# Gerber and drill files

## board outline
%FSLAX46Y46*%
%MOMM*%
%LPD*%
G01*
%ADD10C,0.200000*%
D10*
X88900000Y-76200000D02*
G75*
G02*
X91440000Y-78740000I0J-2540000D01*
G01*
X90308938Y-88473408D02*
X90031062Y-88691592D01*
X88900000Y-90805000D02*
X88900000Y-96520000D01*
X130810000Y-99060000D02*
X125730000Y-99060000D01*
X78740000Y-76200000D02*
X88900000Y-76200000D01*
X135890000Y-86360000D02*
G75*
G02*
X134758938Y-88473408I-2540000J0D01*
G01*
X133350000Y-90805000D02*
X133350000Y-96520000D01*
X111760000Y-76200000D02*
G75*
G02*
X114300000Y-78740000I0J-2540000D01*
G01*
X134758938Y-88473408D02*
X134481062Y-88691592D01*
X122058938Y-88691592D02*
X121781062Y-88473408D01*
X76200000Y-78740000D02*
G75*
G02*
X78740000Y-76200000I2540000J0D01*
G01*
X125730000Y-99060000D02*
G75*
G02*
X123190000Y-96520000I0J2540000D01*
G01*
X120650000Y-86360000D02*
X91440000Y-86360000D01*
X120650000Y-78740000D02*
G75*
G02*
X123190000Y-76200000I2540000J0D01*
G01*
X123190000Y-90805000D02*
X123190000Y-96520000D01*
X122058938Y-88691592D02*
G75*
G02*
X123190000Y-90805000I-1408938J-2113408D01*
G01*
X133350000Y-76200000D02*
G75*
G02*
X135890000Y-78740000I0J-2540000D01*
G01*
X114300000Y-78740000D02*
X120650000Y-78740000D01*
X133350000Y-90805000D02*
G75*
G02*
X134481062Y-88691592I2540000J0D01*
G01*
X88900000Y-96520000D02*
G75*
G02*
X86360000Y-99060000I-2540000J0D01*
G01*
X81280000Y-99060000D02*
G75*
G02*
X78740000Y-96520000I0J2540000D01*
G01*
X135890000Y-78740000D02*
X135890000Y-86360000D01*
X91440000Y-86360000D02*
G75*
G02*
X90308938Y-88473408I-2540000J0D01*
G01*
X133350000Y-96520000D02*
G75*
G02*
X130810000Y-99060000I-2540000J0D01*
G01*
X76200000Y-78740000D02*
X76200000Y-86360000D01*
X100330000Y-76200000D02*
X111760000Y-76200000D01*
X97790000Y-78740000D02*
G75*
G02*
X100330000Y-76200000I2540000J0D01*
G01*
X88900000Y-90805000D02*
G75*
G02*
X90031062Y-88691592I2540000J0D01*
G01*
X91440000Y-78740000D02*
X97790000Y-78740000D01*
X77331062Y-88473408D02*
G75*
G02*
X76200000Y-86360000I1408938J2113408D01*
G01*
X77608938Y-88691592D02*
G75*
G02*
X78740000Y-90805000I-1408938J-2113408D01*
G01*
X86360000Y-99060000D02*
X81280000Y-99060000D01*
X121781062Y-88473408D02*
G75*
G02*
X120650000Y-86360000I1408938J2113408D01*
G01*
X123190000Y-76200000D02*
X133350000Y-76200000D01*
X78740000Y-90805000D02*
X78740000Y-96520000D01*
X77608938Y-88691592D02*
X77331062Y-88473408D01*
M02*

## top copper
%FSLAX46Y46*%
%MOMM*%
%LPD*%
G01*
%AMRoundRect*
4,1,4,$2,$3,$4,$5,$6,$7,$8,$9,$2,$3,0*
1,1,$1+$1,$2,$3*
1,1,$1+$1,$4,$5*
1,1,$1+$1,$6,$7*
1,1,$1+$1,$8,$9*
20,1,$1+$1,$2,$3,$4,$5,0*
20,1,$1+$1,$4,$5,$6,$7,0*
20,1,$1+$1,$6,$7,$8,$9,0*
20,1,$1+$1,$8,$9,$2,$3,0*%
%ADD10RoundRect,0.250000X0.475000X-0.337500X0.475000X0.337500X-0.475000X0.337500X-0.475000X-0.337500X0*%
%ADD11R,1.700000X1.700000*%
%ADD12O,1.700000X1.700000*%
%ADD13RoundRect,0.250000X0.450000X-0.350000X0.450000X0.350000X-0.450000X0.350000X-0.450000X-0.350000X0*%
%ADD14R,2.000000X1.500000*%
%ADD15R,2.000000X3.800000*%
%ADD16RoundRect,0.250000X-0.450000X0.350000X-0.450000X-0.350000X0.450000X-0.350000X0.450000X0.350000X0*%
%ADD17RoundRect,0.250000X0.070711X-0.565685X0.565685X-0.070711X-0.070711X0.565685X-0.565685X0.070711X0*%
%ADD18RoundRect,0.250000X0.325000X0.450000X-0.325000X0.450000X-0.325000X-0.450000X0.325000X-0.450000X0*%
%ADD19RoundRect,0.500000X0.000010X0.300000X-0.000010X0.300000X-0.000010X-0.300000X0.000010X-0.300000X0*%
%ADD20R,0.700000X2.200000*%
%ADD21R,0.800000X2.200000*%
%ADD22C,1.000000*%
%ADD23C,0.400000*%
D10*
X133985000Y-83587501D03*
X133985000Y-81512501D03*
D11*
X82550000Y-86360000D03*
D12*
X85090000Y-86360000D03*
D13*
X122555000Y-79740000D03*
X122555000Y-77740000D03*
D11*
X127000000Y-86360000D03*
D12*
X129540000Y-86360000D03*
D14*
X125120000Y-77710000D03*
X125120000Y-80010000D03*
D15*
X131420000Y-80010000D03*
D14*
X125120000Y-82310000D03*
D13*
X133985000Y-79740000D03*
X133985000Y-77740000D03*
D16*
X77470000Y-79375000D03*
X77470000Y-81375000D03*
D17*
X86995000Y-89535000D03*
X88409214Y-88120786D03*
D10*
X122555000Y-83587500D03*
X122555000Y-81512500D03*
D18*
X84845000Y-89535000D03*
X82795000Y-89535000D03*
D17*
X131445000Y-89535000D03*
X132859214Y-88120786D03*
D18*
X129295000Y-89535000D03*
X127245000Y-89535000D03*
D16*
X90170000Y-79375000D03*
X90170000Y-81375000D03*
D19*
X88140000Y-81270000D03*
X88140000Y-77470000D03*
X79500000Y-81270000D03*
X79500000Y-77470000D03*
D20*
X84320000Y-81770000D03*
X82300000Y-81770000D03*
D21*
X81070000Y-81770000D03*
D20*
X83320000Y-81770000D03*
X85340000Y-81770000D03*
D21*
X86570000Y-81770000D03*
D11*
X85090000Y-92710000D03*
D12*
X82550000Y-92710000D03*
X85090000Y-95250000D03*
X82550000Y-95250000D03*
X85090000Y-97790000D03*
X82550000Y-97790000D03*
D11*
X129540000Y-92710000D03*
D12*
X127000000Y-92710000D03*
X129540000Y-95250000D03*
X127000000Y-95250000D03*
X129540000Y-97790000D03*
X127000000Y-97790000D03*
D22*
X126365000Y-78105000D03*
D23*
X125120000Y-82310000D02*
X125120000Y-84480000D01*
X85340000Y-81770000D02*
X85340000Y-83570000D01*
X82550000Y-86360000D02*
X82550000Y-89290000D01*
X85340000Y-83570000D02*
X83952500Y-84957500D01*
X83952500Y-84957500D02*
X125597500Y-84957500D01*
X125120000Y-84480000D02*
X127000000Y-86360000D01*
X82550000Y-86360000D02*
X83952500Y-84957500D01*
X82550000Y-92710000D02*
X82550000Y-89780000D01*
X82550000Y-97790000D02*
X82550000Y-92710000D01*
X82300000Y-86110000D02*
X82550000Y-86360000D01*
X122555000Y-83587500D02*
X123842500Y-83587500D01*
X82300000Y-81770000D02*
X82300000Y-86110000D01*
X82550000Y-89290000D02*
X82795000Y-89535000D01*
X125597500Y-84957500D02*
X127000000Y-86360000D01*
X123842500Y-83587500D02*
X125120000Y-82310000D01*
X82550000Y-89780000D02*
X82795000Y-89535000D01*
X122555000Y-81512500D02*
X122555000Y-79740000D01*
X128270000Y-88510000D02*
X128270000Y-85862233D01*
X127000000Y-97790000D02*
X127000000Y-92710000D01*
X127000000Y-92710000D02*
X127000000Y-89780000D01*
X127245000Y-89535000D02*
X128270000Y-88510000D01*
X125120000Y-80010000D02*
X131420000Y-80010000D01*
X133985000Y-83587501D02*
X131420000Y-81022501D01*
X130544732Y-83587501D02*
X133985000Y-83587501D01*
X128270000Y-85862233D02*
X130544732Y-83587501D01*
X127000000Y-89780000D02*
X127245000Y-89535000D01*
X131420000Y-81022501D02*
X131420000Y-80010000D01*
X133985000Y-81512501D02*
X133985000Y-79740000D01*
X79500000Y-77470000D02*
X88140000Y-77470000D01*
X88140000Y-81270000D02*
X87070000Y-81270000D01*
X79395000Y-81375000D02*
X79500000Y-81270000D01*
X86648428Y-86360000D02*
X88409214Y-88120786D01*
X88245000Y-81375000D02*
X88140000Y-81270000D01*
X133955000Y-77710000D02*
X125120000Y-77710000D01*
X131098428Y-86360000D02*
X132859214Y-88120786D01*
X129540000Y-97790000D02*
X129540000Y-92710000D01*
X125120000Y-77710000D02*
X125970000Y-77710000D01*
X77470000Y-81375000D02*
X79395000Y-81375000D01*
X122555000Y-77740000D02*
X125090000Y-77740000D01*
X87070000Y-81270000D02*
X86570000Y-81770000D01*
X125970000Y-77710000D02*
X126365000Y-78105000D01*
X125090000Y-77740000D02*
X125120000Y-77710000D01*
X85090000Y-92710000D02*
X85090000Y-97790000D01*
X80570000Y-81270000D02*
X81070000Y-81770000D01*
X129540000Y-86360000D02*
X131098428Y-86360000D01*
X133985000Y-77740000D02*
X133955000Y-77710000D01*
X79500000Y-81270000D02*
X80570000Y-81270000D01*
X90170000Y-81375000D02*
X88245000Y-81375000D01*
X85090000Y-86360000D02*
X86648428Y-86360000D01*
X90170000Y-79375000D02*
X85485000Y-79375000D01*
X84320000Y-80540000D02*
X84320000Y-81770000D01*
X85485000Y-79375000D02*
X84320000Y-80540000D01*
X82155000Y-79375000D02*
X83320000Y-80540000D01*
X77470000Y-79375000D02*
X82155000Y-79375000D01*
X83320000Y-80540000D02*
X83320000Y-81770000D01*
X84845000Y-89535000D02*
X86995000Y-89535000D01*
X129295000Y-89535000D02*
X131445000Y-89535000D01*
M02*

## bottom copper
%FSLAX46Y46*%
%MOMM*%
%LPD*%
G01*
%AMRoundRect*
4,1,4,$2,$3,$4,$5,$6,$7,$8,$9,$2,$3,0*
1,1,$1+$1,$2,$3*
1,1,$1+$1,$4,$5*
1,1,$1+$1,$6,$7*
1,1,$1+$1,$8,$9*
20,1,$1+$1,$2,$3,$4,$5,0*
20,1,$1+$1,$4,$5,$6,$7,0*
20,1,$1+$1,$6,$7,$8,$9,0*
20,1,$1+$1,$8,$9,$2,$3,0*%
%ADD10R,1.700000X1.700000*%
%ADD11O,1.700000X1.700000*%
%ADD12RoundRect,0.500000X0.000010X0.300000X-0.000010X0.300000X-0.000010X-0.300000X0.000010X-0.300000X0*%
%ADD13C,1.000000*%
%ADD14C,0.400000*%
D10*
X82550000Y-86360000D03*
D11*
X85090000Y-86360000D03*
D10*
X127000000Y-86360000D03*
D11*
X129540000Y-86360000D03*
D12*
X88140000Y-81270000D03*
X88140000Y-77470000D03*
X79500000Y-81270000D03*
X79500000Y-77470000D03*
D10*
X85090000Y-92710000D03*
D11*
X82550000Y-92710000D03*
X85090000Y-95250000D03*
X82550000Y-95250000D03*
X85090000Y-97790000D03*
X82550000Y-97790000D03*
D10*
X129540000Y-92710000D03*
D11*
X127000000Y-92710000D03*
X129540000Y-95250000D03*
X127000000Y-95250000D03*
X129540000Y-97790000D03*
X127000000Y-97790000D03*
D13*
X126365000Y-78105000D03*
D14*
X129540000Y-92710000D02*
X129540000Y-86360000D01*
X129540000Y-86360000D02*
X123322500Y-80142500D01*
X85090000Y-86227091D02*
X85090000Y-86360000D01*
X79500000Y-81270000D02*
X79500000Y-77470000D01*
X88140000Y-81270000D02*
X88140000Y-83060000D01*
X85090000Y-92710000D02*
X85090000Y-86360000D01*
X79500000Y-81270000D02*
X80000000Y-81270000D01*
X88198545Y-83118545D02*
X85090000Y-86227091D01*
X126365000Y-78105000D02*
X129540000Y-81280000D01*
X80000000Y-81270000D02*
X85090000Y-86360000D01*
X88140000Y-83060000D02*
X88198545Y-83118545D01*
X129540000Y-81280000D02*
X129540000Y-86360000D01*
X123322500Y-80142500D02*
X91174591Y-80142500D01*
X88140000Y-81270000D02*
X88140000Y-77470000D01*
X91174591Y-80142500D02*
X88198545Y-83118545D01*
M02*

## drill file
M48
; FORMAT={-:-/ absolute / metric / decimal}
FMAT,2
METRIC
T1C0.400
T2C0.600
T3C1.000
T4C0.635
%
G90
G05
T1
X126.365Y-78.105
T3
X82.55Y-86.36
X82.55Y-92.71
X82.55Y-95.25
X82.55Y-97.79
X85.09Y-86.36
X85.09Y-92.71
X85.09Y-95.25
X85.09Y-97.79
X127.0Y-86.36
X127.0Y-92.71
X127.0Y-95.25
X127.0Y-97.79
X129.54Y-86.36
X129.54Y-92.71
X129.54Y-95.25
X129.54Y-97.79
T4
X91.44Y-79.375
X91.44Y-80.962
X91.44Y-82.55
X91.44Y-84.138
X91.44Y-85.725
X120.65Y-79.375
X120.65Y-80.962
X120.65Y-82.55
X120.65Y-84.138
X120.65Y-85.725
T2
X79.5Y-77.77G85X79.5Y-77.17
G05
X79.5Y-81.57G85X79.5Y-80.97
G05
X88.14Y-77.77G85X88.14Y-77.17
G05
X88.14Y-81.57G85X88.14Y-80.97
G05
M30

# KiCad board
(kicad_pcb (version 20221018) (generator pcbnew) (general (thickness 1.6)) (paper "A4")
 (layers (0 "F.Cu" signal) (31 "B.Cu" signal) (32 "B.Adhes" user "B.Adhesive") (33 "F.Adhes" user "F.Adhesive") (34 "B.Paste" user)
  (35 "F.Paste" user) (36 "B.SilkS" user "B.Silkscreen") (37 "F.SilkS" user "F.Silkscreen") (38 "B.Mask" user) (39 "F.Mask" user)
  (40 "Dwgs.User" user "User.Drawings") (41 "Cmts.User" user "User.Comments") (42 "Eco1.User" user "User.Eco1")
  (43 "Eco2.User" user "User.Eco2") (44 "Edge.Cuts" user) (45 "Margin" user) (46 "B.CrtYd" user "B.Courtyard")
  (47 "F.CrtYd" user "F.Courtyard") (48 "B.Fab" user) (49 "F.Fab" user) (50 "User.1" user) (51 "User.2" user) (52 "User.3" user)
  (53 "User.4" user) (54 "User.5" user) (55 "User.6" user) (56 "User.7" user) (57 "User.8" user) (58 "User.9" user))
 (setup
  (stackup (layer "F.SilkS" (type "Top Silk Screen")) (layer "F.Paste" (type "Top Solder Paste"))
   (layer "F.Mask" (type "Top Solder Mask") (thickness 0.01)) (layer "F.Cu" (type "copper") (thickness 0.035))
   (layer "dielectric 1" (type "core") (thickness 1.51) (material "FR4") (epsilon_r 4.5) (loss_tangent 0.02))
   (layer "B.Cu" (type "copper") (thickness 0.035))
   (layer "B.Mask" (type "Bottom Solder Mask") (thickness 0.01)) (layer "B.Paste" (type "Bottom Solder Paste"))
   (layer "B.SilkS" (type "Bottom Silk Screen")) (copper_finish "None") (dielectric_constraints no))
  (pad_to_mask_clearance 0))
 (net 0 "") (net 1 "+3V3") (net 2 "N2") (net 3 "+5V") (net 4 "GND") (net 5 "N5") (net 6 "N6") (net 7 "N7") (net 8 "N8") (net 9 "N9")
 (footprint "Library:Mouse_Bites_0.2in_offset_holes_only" (layer "F.Cu") (at 120.65 82.55 90)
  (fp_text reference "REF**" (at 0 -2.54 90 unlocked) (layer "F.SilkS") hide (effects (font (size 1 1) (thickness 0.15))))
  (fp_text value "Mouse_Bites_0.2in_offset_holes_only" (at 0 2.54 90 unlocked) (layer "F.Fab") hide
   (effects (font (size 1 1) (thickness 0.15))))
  (pad "" np_thru_hole circle (at -3.175 0 90) (size 0.635 0.635) (drill 0.635) (layers "*.Mask") (thermal_bridge_angle 90))
  (pad "" np_thru_hole circle (at -1.5875 0 90) (size 0.635 0.635) (drill 0.635) (layers "*.Mask") (thermal_bridge_angle 90))
  (pad "" np_thru_hole circle (at 0 0 90) (size 0.635 0.635) (drill 0.635) (layers "*.Mask") (thermal_bridge_angle 90))
  (pad "" np_thru_hole circle (at 1.5875 0 90) (size 0.635 0.635) (drill 0.635) (layers "*.Mask") (thermal_bridge_angle 90))
  (pad "" np_thru_hole circle (at 3.175 0 90) (size 0.635 0.635) (drill 0.635) (layers "*.Mask") (thermal_bridge_angle 90)))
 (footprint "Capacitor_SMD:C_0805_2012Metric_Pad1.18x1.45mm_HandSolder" (layer "F.Cu") (at 133.985 82.550001 90)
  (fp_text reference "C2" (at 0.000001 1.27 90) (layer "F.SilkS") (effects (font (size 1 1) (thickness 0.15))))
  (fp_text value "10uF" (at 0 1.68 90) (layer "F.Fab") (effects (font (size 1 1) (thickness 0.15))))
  (pad "1" smd roundrect (at -1.0375 0 90) (size 1.175 1.45) (layers "F.Cu" "F.Paste" "F.Mask") (roundrect_rratio 0.212766) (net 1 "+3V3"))
  (pad "2" smd roundrect (at 1.0375 0 90) (size 1.175 1.45) (layers "F.Cu" "F.Paste" "F.Mask") (roundrect_rratio 0.212766) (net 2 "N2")))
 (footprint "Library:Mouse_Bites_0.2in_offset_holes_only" (layer "F.Cu") (at 91.44 82.55 90)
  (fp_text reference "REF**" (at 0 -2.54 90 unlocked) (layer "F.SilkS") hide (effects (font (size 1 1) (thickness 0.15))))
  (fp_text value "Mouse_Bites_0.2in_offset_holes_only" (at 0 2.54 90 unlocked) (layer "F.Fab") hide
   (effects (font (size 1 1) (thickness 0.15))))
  (pad "" np_thru_hole circle (at -3.175 0 90) (size 0.635 0.635) (drill 0.635) (layers "*.Mask") (thermal_bridge_angle 90))
  (pad "" np_thru_hole circle (at -1.5875 0 90) (size 0.635 0.635) (drill 0.635) (layers "*.Mask") (thermal_bridge_angle 90))
  (pad "" np_thru_hole circle (at 0 0 90) (size 0.635 0.635) (drill 0.635) (layers "*.Mask") (thermal_bridge_angle 90))
  (pad "" np_thru_hole circle (at 1.5875 0 90) (size 0.635 0.635) (drill 0.635) (layers "*.Mask") (thermal_bridge_angle 90))
  (pad "" np_thru_hole circle (at 3.175 0 90) (size 0.635 0.635) (drill 0.635) (layers "*.Mask") (thermal_bridge_angle 90)))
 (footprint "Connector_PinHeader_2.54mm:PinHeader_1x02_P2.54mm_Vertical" (layer "F.Cu") (at 82.55 86.36 90)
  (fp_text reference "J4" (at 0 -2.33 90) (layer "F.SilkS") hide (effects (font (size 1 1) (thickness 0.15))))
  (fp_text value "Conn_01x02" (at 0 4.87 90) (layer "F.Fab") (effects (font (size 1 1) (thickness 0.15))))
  (pad "1" thru_hole rect (at 0 0 90) (size 1.7 1.7) (drill 1) (layers "*.Cu" "*.Mask") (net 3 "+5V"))
  (pad "2" thru_hole oval (at 0 2.54 90) (size 1.7 1.7) (drill 1) (layers "*.Cu" "*.Mask") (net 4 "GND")))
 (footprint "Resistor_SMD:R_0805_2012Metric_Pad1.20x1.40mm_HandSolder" (layer "F.Cu") (at 122.555 78.74 90)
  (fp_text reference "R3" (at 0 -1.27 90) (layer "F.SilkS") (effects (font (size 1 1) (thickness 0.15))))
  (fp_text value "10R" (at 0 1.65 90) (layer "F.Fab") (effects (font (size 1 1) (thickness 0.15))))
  (pad "1" smd roundrect (at -1 0 90) (size 1.2 1.4) (layers "F.Cu" "F.Paste" "F.Mask") (roundrect_rratio 0.208333) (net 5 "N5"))
  (pad "2" smd roundrect (at 1 0 90) (size 1.2 1.4) (layers "F.Cu" "F.Paste" "F.Mask") (roundrect_rratio 0.208333) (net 4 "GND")))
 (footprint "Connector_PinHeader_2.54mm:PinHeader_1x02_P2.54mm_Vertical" (layer "F.Cu") (at 127 86.36 90)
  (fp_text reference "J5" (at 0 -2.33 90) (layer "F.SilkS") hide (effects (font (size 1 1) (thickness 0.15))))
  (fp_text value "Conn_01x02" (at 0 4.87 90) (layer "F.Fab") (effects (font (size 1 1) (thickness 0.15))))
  (pad "1" thru_hole rect (at 0 0 90) (size 1.7 1.7) (drill 1) (layers "*.Cu" "*.Mask") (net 3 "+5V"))
  (pad "2" thru_hole oval (at 0 2.54 90) (size 1.7 1.7) (drill 1) (layers "*.Cu" "*.Mask") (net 4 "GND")))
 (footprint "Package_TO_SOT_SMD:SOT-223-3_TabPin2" (layer "F.Cu") (at 128.27 80.01)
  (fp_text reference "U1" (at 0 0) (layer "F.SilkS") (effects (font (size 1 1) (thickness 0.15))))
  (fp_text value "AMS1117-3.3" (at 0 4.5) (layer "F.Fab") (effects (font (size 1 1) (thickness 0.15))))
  (pad "1" smd rect (at -3.15 -2.3) (size 2 1.5) (layers "F.Cu" "F.Paste" "F.Mask") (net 4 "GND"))
  (pad "2" smd rect (at -3.15 0) (size 2 1.5) (layers "F.Cu" "F.Paste" "F.Mask") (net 1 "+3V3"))
  (pad "2" smd rect (at 3.15 0) (size 2 3.8) (layers "F.Cu" "F.Paste" "F.Mask") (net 1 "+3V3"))
  (pad "3" smd rect (at -3.15 2.3) (size 2 1.5) (layers "F.Cu" "F.Paste" "F.Mask") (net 3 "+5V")))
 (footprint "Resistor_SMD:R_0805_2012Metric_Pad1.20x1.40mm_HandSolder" (layer "F.Cu") (at 133.985 78.74 90)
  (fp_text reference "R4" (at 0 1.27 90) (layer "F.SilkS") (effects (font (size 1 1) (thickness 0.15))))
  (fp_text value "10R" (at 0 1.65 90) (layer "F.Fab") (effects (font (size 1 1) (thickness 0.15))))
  (pad "1" smd roundrect (at -1 0 90) (size 1.2 1.4) (layers "F.Cu" "F.Paste" "F.Mask") (roundrect_rratio 0.208333) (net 2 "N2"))
  (pad "2" smd roundrect (at 1 0 90) (size 1.2 1.4) (layers "F.Cu" "F.Paste" "F.Mask") (roundrect_rratio 0.208333) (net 4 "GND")))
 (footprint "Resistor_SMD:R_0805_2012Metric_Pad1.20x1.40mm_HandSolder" (layer "F.Cu") (at 77.47 80.375 -90)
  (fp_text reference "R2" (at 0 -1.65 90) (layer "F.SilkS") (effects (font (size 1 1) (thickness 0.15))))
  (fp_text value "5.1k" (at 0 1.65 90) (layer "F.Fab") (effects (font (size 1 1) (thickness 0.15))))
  (pad "1" smd roundrect (at -1 0 270) (size 1.2 1.4) (layers "F.Cu" "F.Paste" "F.Mask") (roundrect_rratio 0.208333) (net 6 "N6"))
  (pad "2" smd roundrect (at 1 0 270) (size 1.2 1.4) (layers "F.Cu" "F.Paste" "F.Mask") (roundrect_rratio 0.208333) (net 4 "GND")))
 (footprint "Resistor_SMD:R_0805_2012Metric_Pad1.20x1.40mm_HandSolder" (layer "F.Cu") (at 87.702107 88.827893 45)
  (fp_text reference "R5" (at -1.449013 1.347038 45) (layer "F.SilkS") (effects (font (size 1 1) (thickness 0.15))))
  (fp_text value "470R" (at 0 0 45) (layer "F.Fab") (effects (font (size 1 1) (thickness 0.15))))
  (pad "1" smd roundrect (at -1 0 45) (size 1.2 1.4) (layers "F.Cu" "F.Paste" "F.Mask") (roundrect_rratio 0.208333) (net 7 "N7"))
  (pad "2" smd roundrect (at 1 0 45) (size 1.2 1.4) (layers "F.Cu" "F.Paste" "F.Mask") (roundrect_rratio 0.208333) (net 4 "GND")))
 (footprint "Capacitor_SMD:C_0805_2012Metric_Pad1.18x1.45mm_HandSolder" (layer "F.Cu") (at 122.555 82.55 90)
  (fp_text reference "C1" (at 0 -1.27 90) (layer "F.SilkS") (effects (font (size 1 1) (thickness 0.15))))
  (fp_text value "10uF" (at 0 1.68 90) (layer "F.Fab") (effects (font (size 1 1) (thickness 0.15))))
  (pad "1" smd roundrect (at -1.0375 0 90) (size 1.175 1.45) (layers "F.Cu" "F.Paste" "F.Mask") (roundrect_rratio 0.212766) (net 3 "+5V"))
  (pad "2" smd roundrect (at 1.0375 0 90) (size 1.175 1.45) (layers "F.Cu" "F.Paste" "F.Mask") (roundrect_rratio 0.212766) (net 5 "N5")))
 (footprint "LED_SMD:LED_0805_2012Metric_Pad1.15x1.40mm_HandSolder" (layer "F.Cu") (at 83.82 89.535 180)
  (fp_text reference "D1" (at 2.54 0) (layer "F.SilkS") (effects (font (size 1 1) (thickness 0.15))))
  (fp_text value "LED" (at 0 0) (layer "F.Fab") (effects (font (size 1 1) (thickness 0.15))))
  (pad "1" smd roundrect (at -1.025 0 180) (size 1.15 1.4) (layers "F.Cu" "F.Paste" "F.Mask") (roundrect_rratio 0.217391) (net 7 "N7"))
  (pad "2" smd roundrect (at 1.025 0 180) (size 1.15 1.4) (layers "F.Cu" "F.Paste" "F.Mask") (roundrect_rratio 0.217391) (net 3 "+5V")))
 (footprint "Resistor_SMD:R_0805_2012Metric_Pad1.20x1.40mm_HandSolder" (layer "F.Cu") (at 132.152107 88.827893 45)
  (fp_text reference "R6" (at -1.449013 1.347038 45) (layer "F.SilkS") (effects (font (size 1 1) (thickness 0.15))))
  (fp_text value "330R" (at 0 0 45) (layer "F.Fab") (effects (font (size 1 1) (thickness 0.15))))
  (pad "1" smd roundrect (at -1 0 45) (size 1.2 1.4) (layers "F.Cu" "F.Paste" "F.Mask") (roundrect_rratio 0.208333) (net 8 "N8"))
  (pad "2" smd roundrect (at 1 0 45) (size 1.2 1.4) (layers "F.Cu" "F.Paste" "F.Mask") (roundrect_rratio 0.208333) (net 4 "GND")))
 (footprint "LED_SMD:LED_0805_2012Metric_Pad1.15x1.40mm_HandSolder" (layer "F.Cu") (at 128.27 89.535 180)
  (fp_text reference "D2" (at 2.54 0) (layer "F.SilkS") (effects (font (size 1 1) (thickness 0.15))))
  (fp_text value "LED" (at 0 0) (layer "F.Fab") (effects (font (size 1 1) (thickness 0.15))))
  (pad "1" smd roundrect (at -1.025 0 180) (size 1.15 1.4) (layers "F.Cu" "F.Paste" "F.Mask") (roundrect_rratio 0.217391) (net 8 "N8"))
  (pad "2" smd roundrect (at 1.025 0 180) (size 1.15 1.4) (layers "F.Cu" "F.Paste" "F.Mask") (roundrect_rratio 0.217391) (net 1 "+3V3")))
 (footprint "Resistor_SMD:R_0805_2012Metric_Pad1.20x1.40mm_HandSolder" (layer "F.Cu") (at 90.17 80.375 -90)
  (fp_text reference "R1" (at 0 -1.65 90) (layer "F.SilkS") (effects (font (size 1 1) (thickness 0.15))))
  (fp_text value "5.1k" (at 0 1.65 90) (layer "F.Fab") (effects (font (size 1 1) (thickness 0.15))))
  (pad "1" smd roundrect (at -1 0 270) (size 1.2 1.4) (layers "F.Cu" "F.Paste" "F.Mask") (roundrect_rratio 0.208333) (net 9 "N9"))
  (pad "2" smd roundrect (at 1 0 270) (size 1.2 1.4) (layers "F.Cu" "F.Paste" "F.Mask") (roundrect_rratio 0.208333) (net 4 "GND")))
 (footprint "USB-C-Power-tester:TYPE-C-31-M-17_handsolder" (layer "F.Cu") (at 83.82 77.47 180)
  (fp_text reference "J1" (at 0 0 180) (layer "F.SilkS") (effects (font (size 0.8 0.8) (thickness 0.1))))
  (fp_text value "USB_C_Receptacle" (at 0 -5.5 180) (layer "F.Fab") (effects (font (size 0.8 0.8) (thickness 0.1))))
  (pad "1" thru_hole roundrect (at -4.32 -3.8 180) (size 1 1.6) (drill oval 0.6 1.2) (layers "*.Cu" "*.Mask") (roundrect_rratio 0.5)
   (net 4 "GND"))
  (pad "1" thru_hole roundrect (at -4.32 0 180) (size 1 1.6) (drill oval 0.6 1.2) (layers "*.Cu" "*.Mask") (roundrect_rratio 0.5)
   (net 4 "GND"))
  (pad "1" thru_hole roundrect (at 4.32 -3.8 180) (size 1 1.6) (drill oval 0.6 1.2) (layers "*.Cu" "*.Mask") (roundrect_rratio 0.5)
   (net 4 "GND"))
  (pad "1" thru_hole roundrect (at 4.32 0 180) (size 1 1.6) (drill oval 0.6 1.2) (layers "*.Cu" "*.Mask") (roundrect_rratio 0.5)
   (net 4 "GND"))
  (pad "A5" smd rect (at -0.5 -4.3 180) (size 0.7 2.2) (layers "F.Cu" "F.Paste" "F.Mask") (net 9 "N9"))
  (pad "A9" smd rect (at 1.52 -4.3 180) (size 0.7 2.2) (layers "F.Cu" "F.Paste" "F.Mask") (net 3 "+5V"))
  (pad "A12" smd rect (at 2.75 -4.3 180) (size 0.8 2.2) (layers "F.Cu" "F.Paste" "F.Mask") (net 4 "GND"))
  (pad "B5" smd rect (at 0.5 -4.3 180) (size 0.7 2.2) (layers "F.Cu" "F.Paste" "F.Mask") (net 6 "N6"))
  (pad "B9" smd rect (at -1.52 -4.3 180) (size 0.7 2.2) (layers "F.Cu" "F.Paste" "F.Mask") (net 3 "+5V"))
  (pad "B12" smd rect (at -2.75 -4.3 180) (size 0.8 2.2) (layers "F.Cu" "F.Paste" "F.Mask") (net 4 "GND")))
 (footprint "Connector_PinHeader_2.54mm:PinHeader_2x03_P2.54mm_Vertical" (layer "B.Cu") (at 85.09 92.71 180)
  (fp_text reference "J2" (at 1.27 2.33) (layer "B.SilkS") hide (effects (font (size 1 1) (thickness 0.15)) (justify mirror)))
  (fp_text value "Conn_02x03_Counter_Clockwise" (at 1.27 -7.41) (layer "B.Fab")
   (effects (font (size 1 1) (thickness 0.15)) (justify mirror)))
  (pad "1" thru_hole rect (at 0 0 180) (size 1.7 1.7) (drill 1) (layers "*.Cu" "*.Mask") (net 4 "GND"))
  (pad "2" thru_hole oval (at 2.54 0 180) (size 1.7 1.7) (drill 1) (layers "*.Cu" "*.Mask") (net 3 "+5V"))
  (pad "3" thru_hole oval (at 0 -2.54 180) (size 1.7 1.7) (drill 1) (layers "*.Cu" "*.Mask") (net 4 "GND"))
  (pad "4" thru_hole oval (at 2.54 -2.54 180) (size 1.7 1.7) (drill 1) (layers "*.Cu" "*.Mask") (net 3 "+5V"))
  (pad "5" thru_hole oval (at 0 -5.08 180) (size 1.7 1.7) (drill 1) (layers "*.Cu" "*.Mask") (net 4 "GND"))
  (pad "6" thru_hole oval (at 2.54 -5.08 180) (size 1.7 1.7) (drill 1) (layers "*.Cu" "*.Mask") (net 3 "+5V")))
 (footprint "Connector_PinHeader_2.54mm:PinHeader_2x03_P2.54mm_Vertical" (layer "B.Cu") (at 129.54 92.71 180)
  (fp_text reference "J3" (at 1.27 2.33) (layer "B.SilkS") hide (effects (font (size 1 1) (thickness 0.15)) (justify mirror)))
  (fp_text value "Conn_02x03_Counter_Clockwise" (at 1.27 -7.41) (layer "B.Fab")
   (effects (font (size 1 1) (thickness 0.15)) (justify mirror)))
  (pad "1" thru_hole rect (at 0 0 180) (size 1.7 1.7) (drill 1) (layers "*.Cu" "*.Mask") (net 4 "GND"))
  (pad "2" thru_hole oval (at 2.54 0 180) (size 1.7 1.7) (drill 1) (layers "*.Cu" "*.Mask") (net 1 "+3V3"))
  (pad "3" thru_hole oval (at 0 -2.54 180) (size 1.7 1.7) (drill 1) (layers "*.Cu" "*.Mask") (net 4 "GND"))
  (pad "4" thru_hole oval (at 2.54 -2.54 180) (size 1.7 1.7) (drill 1) (layers "*.Cu" "*.Mask") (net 1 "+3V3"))
  (pad "5" thru_hole oval (at 0 -5.08 180) (size 1.7 1.7) (drill 1) (layers "*.Cu" "*.Mask") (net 4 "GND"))
  (pad "6" thru_hole oval (at 2.54 -5.08 180) (size 1.7 1.7) (drill 1) (layers "*.Cu" "*.Mask") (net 1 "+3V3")))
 (gr_arc (start 88.9 76.2) (mid 90.696051 76.943949) (end 91.44 78.74) (stroke (width 0.2) (type default)) (layer "Edge.Cuts"))
 (gr_line (start 90.308938 88.473408) (end 90.031062 88.691592) (stroke (width 0.2) (type default)) (layer "Edge.Cuts"))
 (gr_line (start 88.9 90.805) (end 88.9 96.52) (stroke (width 0.2) (type default)) (layer "Edge.Cuts"))
 (gr_line (start 130.81 99.06) (end 125.73 99.06) (stroke (width 0.2) (type default)) (layer "Edge.Cuts"))
 (gr_line (start 78.74 76.2) (end 88.9 76.2) (stroke (width 0.2) (type default)) (layer "Edge.Cuts"))
 (gr_arc (start 135.89 86.36) (mid 135.589453 87.558519) (end 134.758938 88.473408) (stroke (width 0.2) (type default)) (layer "Edge.Cuts"))
 (gr_line (start 133.35 90.805) (end 133.35 96.52) (stroke (width 0.2) (type default)) (layer "Edge.Cuts"))
 (gr_arc (start 111.76 76.2) (mid 113.556051 76.943949) (end 114.3 78.74) (stroke (width 0.2) (type default)) (layer "Edge.Cuts"))
 (gr_line (start 134.758938 88.473408) (end 134.481062 88.691592) (stroke (width 0.2) (type default)) (layer "Edge.Cuts"))
 (gr_line (start 122.058938 88.691592) (end 121.781062 88.473408) (stroke (width 0.2) (type default)) (layer "Edge.Cuts"))
 (gr_arc (start 76.2 78.74) (mid 76.943949 76.943949) (end 78.74 76.2) (stroke (width 0.2) (type default)) (layer "Edge.Cuts"))
 (gr_arc (start 125.73 99.06) (mid 123.933949 98.316051) (end 123.19 96.52) (stroke (width 0.2) (type default)) (layer "Edge.Cuts"))
 (gr_line (start 120.65 86.36) (end 91.44 86.36) (stroke (width 0.2) (type default)) (layer "Edge.Cuts"))
 (gr_arc (start 120.65 78.74) (mid 121.393949 76.943949) (end 123.19 76.2) (stroke (width 0.2) (type default)) (layer "Edge.Cuts"))
 (gr_line (start 123.19 90.805) (end 123.19 96.52) (stroke (width 0.2) (type default)) (layer "Edge.Cuts"))
 (gr_arc (start 122.058938 88.691592) (mid 122.889453 89.606481) (end 123.19 90.805) (stroke (width 0.2) (type default)) (layer "Edge.Cuts"))
 (gr_arc (start 133.35 76.2) (mid 135.146051 76.943949) (end 135.89 78.74) (stroke (width 0.2) (type default)) (layer "Edge.Cuts"))
 (gr_line (start 114.3 78.74) (end 120.65 78.74) (stroke (width 0.2) (type default)) (layer "Edge.Cuts"))
 (gr_arc (start 133.35 90.805) (mid 133.650547 89.606481) (end 134.481062 88.691592) (stroke (width 0.2) (type default)) (layer "Edge.Cuts"))
 (gr_arc (start 88.9 96.52) (mid 88.156051 98.316051) (end 86.36 99.06) (stroke (width 0.2) (type default)) (layer "Edge.Cuts"))
 (gr_arc (start 81.28 99.06) (mid 79.483949 98.316051) (end 78.74 96.52) (stroke (width 0.2) (type default)) (layer "Edge.Cuts"))
 (gr_line (start 135.89 78.74) (end 135.89 86.36) (stroke (width 0.2) (type default)) (layer "Edge.Cuts"))
 (gr_arc (start 91.44 86.36) (mid 91.139453 87.558519) (end 90.308938 88.473408) (stroke (width 0.2) (type default)) (layer "Edge.Cuts"))
 (gr_arc (start 133.35 96.52) (mid 132.606051 98.316051) (end 130.81 99.06) (stroke (width 0.2) (type default)) (layer "Edge.Cuts"))
 (gr_line (start 76.2 78.74) (end 76.2 86.36) (stroke (width 0.2) (type default)) (layer "Edge.Cuts"))
 (gr_line (start 100.33 76.2) (end 111.76 76.2) (stroke (width 0.2) (type default)) (layer "Edge.Cuts"))
 (gr_arc (start 97.79 78.74) (mid 98.533949 76.943949) (end 100.33 76.2) (stroke (width 0.2) (type default)) (layer "Edge.Cuts"))
 (gr_arc (start 88.9 90.805) (mid 89.200547 89.606481) (end 90.031062 88.691592) (stroke (width 0.2) (type default)) (layer "Edge.Cuts"))
 (gr_line (start 91.44 78.74) (end 97.79 78.74) (stroke (width 0.2) (type default)) (layer "Edge.Cuts"))
 (gr_arc (start 77.331062 88.473408) (mid 76.500547 87.558519) (end 76.2 86.36) (stroke (width 0.2) (type default)) (layer "Edge.Cuts"))
 (gr_arc (start 77.608938 88.691592) (mid 78.439453 89.606481) (end 78.74 90.805) (stroke (width 0.2) (type default)) (layer "Edge.Cuts"))
 (gr_line (start 86.36 99.06) (end 81.28 99.06) (stroke (width 0.2) (type default)) (layer "Edge.Cuts"))
 (gr_arc (start 121.781062 88.473408) (mid 120.950547 87.558519) (end 120.65 86.36) (stroke (width 0.2) (type default)) (layer "Edge.Cuts"))
 (gr_line (start 123.19 76.2) (end 133.35 76.2) (stroke (width 0.2) (type default)) (layer "Edge.Cuts"))
 (gr_line (start 78.74 90.805) (end 78.74 96.52) (stroke (width 0.2) (type default)) (layer "Edge.Cuts"))
 (gr_line (start 77.608938 88.691592) (end 77.331062 88.473408) (stroke (width 0.2) (type default)) (layer "Edge.Cuts"))
 (segment (start 125.12 82.31) (end 125.12 84.48) (width 0.4) (layer "F.Cu") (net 3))
 (segment (start 85.34 81.77) (end 85.34 83.57) (width 0.4) (layer "F.Cu") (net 3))
 (segment (start 82.55 86.36) (end 82.55 89.29) (width 0.4) (layer "F.Cu") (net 3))
 (segment (start 85.34 83.57) (end 83.9525 84.9575) (width 0.4) (layer "F.Cu") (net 3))
 (segment (start 83.9525 84.9575) (end 125.5975 84.9575) (width 0.4) (layer "F.Cu") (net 3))
 (segment (start 125.12 84.48) (end 127 86.36) (width 0.4) (layer "F.Cu") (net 3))
 (segment (start 82.55 86.36) (end 83.9525 84.9575) (width 0.4) (layer "F.Cu") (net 3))
 (segment (start 82.55 92.71) (end 82.55 89.78) (width 0.4) (layer "F.Cu") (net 3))
 (segment (start 82.55 97.79) (end 82.55 92.71) (width 0.4) (layer "F.Cu") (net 3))
 (segment (start 82.3 86.11) (end 82.55 86.36) (width 0.4) (layer "F.Cu") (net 3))
 (segment (start 122.555 83.5875) (end 123.8425 83.5875) (width 0.4) (layer "F.Cu") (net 3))
 (segment (start 82.3 81.77) (end 82.3 86.11) (width 0.4) (layer "F.Cu") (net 3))
 (segment (start 82.55 89.29) (end 82.795 89.535) (width 0.4) (layer "F.Cu") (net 3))
 (segment (start 125.5975 84.9575) (end 127 86.36) (width 0.4) (layer "F.Cu") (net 3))
 (segment (start 123.8425 83.5875) (end 125.12 82.31) (width 0.4) (layer "F.Cu") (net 3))
 (segment (start 82.55 89.78) (end 82.795 89.535) (width 0.4) (layer "F.Cu") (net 3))
 (segment (start 122.555 81.5125) (end 122.555 79.74) (width 0.4) (layer "F.Cu") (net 5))
 (segment (start 128.27 88.51) (end 128.27 85.862233) (width 0.4) (layer "F.Cu") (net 1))
 (segment (start 127 97.79) (end 127 92.71) (width 0.4) (layer "F.Cu") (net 1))
 (segment (start 127 92.71) (end 127 89.78) (width 0.4) (layer "F.Cu") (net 1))
 (segment (start 127.245 89.535) (end 128.27 88.51) (width 0.4) (layer "F.Cu") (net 1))
 (segment (start 125.12 80.01) (end 131.42 80.01) (width 0.4) (layer "F.Cu") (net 1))
 (segment (start 133.985 83.587501) (end 131.42 81.022501) (width 0.4) (layer "F.Cu") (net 1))
 (segment (start 130.544732 83.587501) (end 133.985 83.587501) (width 0.4) (layer "F.Cu") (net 1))
 (segment (start 128.27 85.862233) (end 130.544732 83.587501) (width 0.4) (layer "F.Cu") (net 1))
 (segment (start 127 89.78) (end 127.245 89.535) (width 0.4) (layer "F.Cu") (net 1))
 (segment (start 131.42 81.022501) (end 131.42 80.01) (width 0.4) (layer "F.Cu") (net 1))
 (segment (start 133.985 81.512501) (end 133.985 79.74) (width 0.4) (layer "F.Cu") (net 2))
 (segment (start 79.5 77.47) (end 88.14 77.47) (width 0.4) (layer "F.Cu") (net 4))
 (segment (start 88.14 81.27) (end 87.07 81.27) (width 0.4) (layer "F.Cu") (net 4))
 (segment (start 79.395 81.375) (end 79.5 81.27) (width 0.4) (layer "F.Cu") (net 4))
 (segment (start 86.648428 86.36) (end 88.409214 88.120786) (width 0.4) (layer "F.Cu") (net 4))
 (segment (start 88.245 81.375) (end 88.14 81.27) (width 0.4) (layer "F.Cu") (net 4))
 (segment (start 133.955 77.71) (end 125.12 77.71) (width 0.4) (layer "F.Cu") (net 4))
 (segment (start 131.098428 86.36) (end 132.859214 88.120786) (width 0.4) (layer "F.Cu") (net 4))
 (segment (start 129.54 97.79) (end 129.54 92.71) (width 0.4) (layer "F.Cu") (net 4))
 (segment (start 125.12 77.71) (end 125.97 77.71) (width 0.4) (layer "F.Cu") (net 4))
 (segment (start 77.47 81.375) (end 79.395 81.375) (width 0.4) (layer "F.Cu") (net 4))
 (segment (start 122.555 77.74) (end 125.09 77.74) (width 0.4) (layer "F.Cu") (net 4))
 (segment (start 87.07 81.27) (end 86.57 81.77) (width 0.4) (layer "F.Cu") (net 4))
 (segment (start 125.97 77.71) (end 126.365 78.105) (width 0.4) (layer "F.Cu") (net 4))
 (segment (start 125.09 77.74) (end 125.12 77.71) (width 0.4) (layer "F.Cu") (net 4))
 (segment (start 85.09 92.71) (end 85.09 97.79) (width 0.4) (layer "F.Cu") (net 4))
 (segment (start 80.57 81.27) (end 81.07 81.77) (width 0.4) (layer "F.Cu") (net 4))
 (segment (start 129.54 86.36) (end 131.098428 86.36) (width 0.4) (layer "F.Cu") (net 4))
 (segment (start 133.985 77.74) (end 133.955 77.71) (width 0.4) (layer "F.Cu") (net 4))
 (segment (start 79.5 81.27) (end 80.57 81.27) (width 0.4) (layer "F.Cu") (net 4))
 (segment (start 90.17 81.375) (end 88.245 81.375) (width 0.4) (layer "F.Cu") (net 4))
 (segment (start 85.09 86.36) (end 86.648428 86.36) (width 0.4) (layer "F.Cu") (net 4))
 (via (at 126.365 78.105) (size 1) (drill 0.4) (layers "F.Cu" "B.Cu") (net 4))
 (segment (start 129.54 92.71) (end 129.54 86.36) (width 0.4) (layer "B.Cu") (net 4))
 (segment (start 129.54 86.36) (end 123.3225 80.1425) (width 0.4) (layer "B.Cu") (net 4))
 (segment (start 85.09 86.227091) (end 85.09 86.36) (width 0.4) (layer "B.Cu") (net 4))
 (segment (start 79.5 81.27) (end 79.5 77.47) (width 0.4) (layer "B.Cu") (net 4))
 (segment (start 88.14 81.27) (end 88.14 83.06) (width 0.4) (layer "B.Cu") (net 4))
 (segment (start 85.09 92.71) (end 85.09 86.36) (width 0.4) (layer "B.Cu") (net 4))
 (segment (start 79.5 81.27) (end 80 81.27) (width 0.4) (layer "B.Cu") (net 4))
 (segment (start 88.198545 83.118545) (end 85.09 86.227091) (width 0.4) (layer "B.Cu") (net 4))
 (segment (start 126.365 78.105) (end 129.54 81.28) (width 0.4) (layer "B.Cu") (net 4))
 (segment (start 80 81.27) (end 85.09 86.36) (width 0.4) (layer "B.Cu") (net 4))
 (segment (start 88.14 83.06) (end 88.198545 83.118545) (width 0.4) (layer "B.Cu") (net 4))
 (segment (start 129.54 81.28) (end 129.54 86.36) (width 0.4) (layer "B.Cu") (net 4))
 (segment (start 123.3225 80.1425) (end 91.174591 80.1425) (width 0.4) (layer "B.Cu") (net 4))
 (segment (start 88.14 81.27) (end 88.14 77.47) (width 0.4) (layer "B.Cu") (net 4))
 (segment (start 91.174591 80.1425) (end 88.198545 83.118545) (width 0.4) (layer "B.Cu") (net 4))
 (segment (start 90.17 79.375) (end 85.485 79.375) (width 0.4) (layer "F.Cu") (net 9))
 (segment (start 84.32 80.54) (end 84.32 81.77) (width 0.4) (layer "F.Cu") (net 9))
 (segment (start 85.485 79.375) (end 84.32 80.54) (width 0.4) (layer "F.Cu") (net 9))
 (segment (start 82.155 79.375) (end 83.32 80.54) (width 0.4) (layer "F.Cu") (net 6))
 (segment (start 77.47 79.375) (end 82.155 79.375) (width 0.4) (layer "F.Cu") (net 6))
 (segment (start 83.32 80.54) (end 83.32 81.77) (width 0.4) (layer "F.Cu") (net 6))
 (segment (start 84.845 89.535) (end 86.995 89.535) (width 0.4) (layer "F.Cu") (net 7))
 (segment (start 129.295 89.535) (end 131.445 89.535) (width 0.4) (layer "F.Cu") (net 8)))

